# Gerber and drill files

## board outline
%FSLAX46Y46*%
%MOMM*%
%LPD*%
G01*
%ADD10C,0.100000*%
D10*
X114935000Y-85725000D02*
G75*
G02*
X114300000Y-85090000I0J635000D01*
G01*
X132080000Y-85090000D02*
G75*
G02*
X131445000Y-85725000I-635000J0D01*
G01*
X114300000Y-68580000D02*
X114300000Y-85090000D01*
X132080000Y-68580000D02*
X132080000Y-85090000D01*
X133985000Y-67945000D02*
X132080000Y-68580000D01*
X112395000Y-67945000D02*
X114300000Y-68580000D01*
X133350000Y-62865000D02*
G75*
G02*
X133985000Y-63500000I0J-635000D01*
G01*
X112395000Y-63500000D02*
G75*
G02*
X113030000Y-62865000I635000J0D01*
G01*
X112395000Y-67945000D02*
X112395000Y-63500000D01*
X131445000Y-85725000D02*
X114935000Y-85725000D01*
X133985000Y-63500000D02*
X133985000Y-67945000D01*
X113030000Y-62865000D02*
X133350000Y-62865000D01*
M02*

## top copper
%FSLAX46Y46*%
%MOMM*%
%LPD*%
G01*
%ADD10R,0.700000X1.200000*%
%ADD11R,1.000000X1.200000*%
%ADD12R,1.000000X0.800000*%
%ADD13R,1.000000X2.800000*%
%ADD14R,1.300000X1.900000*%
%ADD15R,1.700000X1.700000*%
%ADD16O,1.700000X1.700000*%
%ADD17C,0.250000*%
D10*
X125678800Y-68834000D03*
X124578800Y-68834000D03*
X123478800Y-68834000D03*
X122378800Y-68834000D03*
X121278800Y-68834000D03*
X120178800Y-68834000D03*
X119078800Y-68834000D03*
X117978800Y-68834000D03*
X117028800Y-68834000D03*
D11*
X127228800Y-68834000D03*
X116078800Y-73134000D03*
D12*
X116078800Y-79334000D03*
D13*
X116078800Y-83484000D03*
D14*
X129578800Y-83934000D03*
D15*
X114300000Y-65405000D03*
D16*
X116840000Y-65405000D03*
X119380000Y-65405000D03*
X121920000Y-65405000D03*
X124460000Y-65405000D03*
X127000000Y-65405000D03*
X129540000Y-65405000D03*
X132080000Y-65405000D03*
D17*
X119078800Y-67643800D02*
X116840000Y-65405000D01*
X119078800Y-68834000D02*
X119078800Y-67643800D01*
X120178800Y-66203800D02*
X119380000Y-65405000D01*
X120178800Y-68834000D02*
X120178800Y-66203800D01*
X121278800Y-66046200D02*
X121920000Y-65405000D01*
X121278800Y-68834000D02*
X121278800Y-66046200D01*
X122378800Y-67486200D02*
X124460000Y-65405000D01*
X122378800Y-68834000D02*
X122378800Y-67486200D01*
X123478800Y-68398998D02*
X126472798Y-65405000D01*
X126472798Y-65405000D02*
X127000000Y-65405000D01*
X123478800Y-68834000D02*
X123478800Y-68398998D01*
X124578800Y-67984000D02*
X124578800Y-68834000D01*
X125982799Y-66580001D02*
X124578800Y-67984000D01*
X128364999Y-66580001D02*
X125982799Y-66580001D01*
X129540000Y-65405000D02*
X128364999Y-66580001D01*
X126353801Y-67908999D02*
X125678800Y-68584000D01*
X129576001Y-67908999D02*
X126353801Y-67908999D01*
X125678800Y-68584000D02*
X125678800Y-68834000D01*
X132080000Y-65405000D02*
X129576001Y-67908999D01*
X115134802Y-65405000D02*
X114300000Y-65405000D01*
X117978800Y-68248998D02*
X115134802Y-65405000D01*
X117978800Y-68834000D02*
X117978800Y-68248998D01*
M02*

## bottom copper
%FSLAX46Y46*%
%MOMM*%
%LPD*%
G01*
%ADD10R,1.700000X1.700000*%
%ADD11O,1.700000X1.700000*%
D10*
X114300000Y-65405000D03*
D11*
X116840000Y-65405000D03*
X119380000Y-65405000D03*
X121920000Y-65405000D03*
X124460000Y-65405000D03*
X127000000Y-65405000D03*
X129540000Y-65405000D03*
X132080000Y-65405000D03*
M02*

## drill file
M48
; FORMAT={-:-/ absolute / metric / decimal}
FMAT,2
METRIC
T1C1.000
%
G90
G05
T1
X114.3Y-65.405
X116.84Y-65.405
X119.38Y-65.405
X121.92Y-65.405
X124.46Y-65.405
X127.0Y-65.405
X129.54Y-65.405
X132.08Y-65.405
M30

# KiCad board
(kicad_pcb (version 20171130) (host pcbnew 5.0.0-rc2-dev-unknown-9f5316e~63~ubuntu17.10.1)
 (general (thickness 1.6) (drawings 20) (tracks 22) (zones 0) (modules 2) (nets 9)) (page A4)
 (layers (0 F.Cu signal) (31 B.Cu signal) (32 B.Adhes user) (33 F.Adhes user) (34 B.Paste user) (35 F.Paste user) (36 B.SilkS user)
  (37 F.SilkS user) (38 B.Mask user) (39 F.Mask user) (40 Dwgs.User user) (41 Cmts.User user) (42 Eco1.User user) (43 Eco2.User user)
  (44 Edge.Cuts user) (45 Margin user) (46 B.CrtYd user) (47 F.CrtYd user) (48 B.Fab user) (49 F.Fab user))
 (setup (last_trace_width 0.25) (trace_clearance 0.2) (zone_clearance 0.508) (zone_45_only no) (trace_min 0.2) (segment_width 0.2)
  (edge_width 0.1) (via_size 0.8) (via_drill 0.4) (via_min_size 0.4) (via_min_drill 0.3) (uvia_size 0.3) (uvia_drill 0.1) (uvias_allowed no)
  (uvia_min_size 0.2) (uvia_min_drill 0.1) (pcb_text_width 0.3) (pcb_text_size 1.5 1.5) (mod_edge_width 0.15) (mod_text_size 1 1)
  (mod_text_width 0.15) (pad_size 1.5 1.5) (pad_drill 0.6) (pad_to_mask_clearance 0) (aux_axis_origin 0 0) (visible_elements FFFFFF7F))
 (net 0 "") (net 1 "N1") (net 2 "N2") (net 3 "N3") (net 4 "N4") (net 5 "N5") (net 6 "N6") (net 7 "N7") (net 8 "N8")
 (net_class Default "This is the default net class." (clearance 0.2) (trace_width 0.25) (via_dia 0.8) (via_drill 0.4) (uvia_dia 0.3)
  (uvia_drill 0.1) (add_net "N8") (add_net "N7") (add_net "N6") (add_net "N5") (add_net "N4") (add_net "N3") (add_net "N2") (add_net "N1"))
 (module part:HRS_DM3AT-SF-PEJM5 (layer F.Cu) (at 122.4788 68.834)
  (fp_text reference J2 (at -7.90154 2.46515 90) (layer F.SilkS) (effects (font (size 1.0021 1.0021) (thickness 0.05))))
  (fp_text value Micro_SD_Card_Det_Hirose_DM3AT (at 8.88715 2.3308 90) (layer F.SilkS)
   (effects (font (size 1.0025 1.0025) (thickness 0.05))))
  (pad 1 smd rect (at 3.2 0) (size 0.7 1.2) (layers F.Cu F.Paste F.Mask) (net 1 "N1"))
  (pad 2 smd rect (at 2.1 0) (size 0.7 1.2) (layers F.Cu F.Paste F.Mask) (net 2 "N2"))
  (pad 3 smd rect (at 1 0) (size 0.7 1.2) (layers F.Cu F.Paste F.Mask) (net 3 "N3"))
  (pad 4 smd rect (at -0.1 0) (size 0.7 1.2) (layers F.Cu F.Paste F.Mask) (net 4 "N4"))
  (pad 5 smd rect (at -1.2 0) (size 0.7 1.2) (layers F.Cu F.Paste F.Mask) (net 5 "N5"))
  (pad 6 smd rect (at -2.3 0) (size 0.7 1.2) (layers F.Cu F.Paste F.Mask) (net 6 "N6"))
  (pad 7 smd rect (at -3.4 0) (size 0.7 1.2) (layers F.Cu F.Paste F.Mask) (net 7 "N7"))
  (pad 8 smd rect (at -4.5 0) (size 0.7 1.2) (layers F.Cu F.Paste F.Mask) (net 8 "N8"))
  (pad SWB smd rect (at -5.45 0) (size 0.7 1.2) (layers F.Cu F.Paste F.Mask))
  (pad P4 smd rect (at 4.75 0) (size 1 1.2) (layers F.Cu F.Paste F.Mask))
  (pad P1 smd rect (at -6.4 4.3) (size 1 1.2) (layers F.Cu F.Paste F.Mask))
  (pad SWA smd rect (at -6.4 10.5) (size 1 0.8) (layers F.Cu F.Paste F.Mask))
  (pad P2 smd rect (at -6.4 14.65) (size 1 2.8) (layers F.Cu F.Paste F.Mask))
  (pad P3 smd rect (at 7.1 15.1) (size 1.3 1.9) (layers F.Cu F.Paste F.Mask)))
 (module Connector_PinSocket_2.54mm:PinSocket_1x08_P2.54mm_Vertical (layer F.Cu) (at 114.3 65.405 90)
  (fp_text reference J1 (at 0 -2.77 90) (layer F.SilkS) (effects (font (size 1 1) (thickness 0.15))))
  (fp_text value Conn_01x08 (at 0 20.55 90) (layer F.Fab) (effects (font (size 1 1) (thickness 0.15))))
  (pad 1 thru_hole rect (at 0 0 90) (size 1.7 1.7) (drill 1) (layers *.Cu *.Mask) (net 8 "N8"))
  (pad 2 thru_hole oval (at 0 2.54 90) (size 1.7 1.7) (drill 1) (layers *.Cu *.Mask) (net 7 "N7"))
  (pad 3 thru_hole oval (at 0 5.08 90) (size 1.7 1.7) (drill 1) (layers *.Cu *.Mask) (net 6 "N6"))
  (pad 4 thru_hole oval (at 0 7.62 90) (size 1.7 1.7) (drill 1) (layers *.Cu *.Mask) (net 5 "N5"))
  (pad 5 thru_hole oval (at 0 10.16 90) (size 1.7 1.7) (drill 1) (layers *.Cu *.Mask) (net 4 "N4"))
  (pad 6 thru_hole oval (at 0 12.7 90) (size 1.7 1.7) (drill 1) (layers *.Cu *.Mask) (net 3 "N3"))
  (pad 7 thru_hole oval (at 0 15.24 90) (size 1.7 1.7) (drill 1) (layers *.Cu *.Mask) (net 2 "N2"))
  (pad 8 thru_hole oval (at 0 17.78 90) (size 1.7 1.7) (drill 1) (layers *.Cu *.Mask) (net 1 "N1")))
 (gr_arc (start 114.935 85.09) (end 114.3 85.09) (angle -90) (layer Edge.Cuts) (width 0.1))
 (gr_arc (start 131.445 85.09) (end 131.445 85.725) (angle -90) (layer Edge.Cuts) (width 0.1))
 (gr_line (start 114.3 68.58) (end 114.3 85.09) (layer Edge.Cuts) (width 0.1))
 (gr_line (start 132.08 68.58) (end 132.08 85.09) (layer Edge.Cuts) (width 0.1))
 (gr_line (start 133.985 67.945) (end 132.08 68.58) (layer Edge.Cuts) (width 0.1))
 (gr_line (start 112.395 67.945) (end 114.3 68.58) (layer Edge.Cuts) (width 0.1))
 (gr_arc (start 133.35 63.5) (end 133.985 63.5) (angle -90) (layer Edge.Cuts) (width 0.1))
 (gr_arc (start 113.03 63.5) (end 113.03 62.865) (angle -90) (layer Edge.Cuts) (width 0.1))
 (gr_line (start 112.395 67.945) (end 112.395 63.5) (layer Edge.Cuts) (width 0.1))
 (gr_line (start 131.445 85.725) (end 114.935 85.725) (layer Edge.Cuts) (width 0.1))
 (gr_line (start 133.985 63.5) (end 133.985 67.945) (layer Edge.Cuts) (width 0.1))
 (gr_line (start 113.03 62.865) (end 133.35 62.865) (layer Edge.Cuts) (width 0.1))
 (segment (start 119.0788 67.6438) (end 116.84 65.405) (width 0.25) (layer F.Cu) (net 7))
 (segment (start 119.0788 68.834) (end 119.0788 67.6438) (width 0.25) (layer F.Cu) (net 7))
 (segment (start 120.1788 66.2038) (end 119.38 65.405) (width 0.25) (layer F.Cu) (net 6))
 (segment (start 120.1788 68.834) (end 120.1788 66.2038) (width 0.25) (layer F.Cu) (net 6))
 (segment (start 121.2788 66.0462) (end 121.92 65.405) (width 0.25) (layer F.Cu) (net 5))
 (segment (start 121.2788 68.834) (end 121.2788 66.0462) (width 0.25) (layer F.Cu) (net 5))
 (segment (start 122.3788 67.4862) (end 124.46 65.405) (width 0.25) (layer F.Cu) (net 4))
 (segment (start 122.3788 68.834) (end 122.3788 67.4862) (width 0.25) (layer F.Cu) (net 4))
 (segment (start 123.4788 68.398998) (end 126.472798 65.405) (width 0.25) (layer F.Cu) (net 3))
 (segment (start 126.472798 65.405) (end 127 65.405) (width 0.25) (layer F.Cu) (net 3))
 (segment (start 123.4788 68.834) (end 123.4788 68.398998) (width 0.25) (layer F.Cu) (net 3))
 (segment (start 124.5788 67.984) (end 124.5788 68.834) (width 0.25) (layer F.Cu) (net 2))
 (segment (start 125.982799 66.580001) (end 124.5788 67.984) (width 0.25) (layer F.Cu) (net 2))
 (segment (start 128.364999 66.580001) (end 125.982799 66.580001) (width 0.25) (layer F.Cu) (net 2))
 (segment (start 129.54 65.405) (end 128.364999 66.580001) (width 0.25) (layer F.Cu) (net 2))
 (segment (start 126.353801 67.908999) (end 125.6788 68.584) (width 0.25) (layer F.Cu) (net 1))
 (segment (start 129.576001 67.908999) (end 126.353801 67.908999) (width 0.25) (layer F.Cu) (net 1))
 (segment (start 125.6788 68.584) (end 125.6788 68.834) (width 0.25) (layer F.Cu) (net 1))
 (segment (start 132.08 65.405) (end 129.576001 67.908999) (width 0.25) (layer F.Cu) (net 1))
 (segment (start 115.134802 65.405) (end 114.3 65.405) (width 0.25) (layer F.Cu) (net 8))
 (segment (start 117.9788 68.248998) (end 115.134802 65.405) (width 0.25) (layer F.Cu) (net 8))
 (segment (start 117.9788 68.834) (end 117.9788 68.248998) (width 0.25) (layer F.Cu) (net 8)))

